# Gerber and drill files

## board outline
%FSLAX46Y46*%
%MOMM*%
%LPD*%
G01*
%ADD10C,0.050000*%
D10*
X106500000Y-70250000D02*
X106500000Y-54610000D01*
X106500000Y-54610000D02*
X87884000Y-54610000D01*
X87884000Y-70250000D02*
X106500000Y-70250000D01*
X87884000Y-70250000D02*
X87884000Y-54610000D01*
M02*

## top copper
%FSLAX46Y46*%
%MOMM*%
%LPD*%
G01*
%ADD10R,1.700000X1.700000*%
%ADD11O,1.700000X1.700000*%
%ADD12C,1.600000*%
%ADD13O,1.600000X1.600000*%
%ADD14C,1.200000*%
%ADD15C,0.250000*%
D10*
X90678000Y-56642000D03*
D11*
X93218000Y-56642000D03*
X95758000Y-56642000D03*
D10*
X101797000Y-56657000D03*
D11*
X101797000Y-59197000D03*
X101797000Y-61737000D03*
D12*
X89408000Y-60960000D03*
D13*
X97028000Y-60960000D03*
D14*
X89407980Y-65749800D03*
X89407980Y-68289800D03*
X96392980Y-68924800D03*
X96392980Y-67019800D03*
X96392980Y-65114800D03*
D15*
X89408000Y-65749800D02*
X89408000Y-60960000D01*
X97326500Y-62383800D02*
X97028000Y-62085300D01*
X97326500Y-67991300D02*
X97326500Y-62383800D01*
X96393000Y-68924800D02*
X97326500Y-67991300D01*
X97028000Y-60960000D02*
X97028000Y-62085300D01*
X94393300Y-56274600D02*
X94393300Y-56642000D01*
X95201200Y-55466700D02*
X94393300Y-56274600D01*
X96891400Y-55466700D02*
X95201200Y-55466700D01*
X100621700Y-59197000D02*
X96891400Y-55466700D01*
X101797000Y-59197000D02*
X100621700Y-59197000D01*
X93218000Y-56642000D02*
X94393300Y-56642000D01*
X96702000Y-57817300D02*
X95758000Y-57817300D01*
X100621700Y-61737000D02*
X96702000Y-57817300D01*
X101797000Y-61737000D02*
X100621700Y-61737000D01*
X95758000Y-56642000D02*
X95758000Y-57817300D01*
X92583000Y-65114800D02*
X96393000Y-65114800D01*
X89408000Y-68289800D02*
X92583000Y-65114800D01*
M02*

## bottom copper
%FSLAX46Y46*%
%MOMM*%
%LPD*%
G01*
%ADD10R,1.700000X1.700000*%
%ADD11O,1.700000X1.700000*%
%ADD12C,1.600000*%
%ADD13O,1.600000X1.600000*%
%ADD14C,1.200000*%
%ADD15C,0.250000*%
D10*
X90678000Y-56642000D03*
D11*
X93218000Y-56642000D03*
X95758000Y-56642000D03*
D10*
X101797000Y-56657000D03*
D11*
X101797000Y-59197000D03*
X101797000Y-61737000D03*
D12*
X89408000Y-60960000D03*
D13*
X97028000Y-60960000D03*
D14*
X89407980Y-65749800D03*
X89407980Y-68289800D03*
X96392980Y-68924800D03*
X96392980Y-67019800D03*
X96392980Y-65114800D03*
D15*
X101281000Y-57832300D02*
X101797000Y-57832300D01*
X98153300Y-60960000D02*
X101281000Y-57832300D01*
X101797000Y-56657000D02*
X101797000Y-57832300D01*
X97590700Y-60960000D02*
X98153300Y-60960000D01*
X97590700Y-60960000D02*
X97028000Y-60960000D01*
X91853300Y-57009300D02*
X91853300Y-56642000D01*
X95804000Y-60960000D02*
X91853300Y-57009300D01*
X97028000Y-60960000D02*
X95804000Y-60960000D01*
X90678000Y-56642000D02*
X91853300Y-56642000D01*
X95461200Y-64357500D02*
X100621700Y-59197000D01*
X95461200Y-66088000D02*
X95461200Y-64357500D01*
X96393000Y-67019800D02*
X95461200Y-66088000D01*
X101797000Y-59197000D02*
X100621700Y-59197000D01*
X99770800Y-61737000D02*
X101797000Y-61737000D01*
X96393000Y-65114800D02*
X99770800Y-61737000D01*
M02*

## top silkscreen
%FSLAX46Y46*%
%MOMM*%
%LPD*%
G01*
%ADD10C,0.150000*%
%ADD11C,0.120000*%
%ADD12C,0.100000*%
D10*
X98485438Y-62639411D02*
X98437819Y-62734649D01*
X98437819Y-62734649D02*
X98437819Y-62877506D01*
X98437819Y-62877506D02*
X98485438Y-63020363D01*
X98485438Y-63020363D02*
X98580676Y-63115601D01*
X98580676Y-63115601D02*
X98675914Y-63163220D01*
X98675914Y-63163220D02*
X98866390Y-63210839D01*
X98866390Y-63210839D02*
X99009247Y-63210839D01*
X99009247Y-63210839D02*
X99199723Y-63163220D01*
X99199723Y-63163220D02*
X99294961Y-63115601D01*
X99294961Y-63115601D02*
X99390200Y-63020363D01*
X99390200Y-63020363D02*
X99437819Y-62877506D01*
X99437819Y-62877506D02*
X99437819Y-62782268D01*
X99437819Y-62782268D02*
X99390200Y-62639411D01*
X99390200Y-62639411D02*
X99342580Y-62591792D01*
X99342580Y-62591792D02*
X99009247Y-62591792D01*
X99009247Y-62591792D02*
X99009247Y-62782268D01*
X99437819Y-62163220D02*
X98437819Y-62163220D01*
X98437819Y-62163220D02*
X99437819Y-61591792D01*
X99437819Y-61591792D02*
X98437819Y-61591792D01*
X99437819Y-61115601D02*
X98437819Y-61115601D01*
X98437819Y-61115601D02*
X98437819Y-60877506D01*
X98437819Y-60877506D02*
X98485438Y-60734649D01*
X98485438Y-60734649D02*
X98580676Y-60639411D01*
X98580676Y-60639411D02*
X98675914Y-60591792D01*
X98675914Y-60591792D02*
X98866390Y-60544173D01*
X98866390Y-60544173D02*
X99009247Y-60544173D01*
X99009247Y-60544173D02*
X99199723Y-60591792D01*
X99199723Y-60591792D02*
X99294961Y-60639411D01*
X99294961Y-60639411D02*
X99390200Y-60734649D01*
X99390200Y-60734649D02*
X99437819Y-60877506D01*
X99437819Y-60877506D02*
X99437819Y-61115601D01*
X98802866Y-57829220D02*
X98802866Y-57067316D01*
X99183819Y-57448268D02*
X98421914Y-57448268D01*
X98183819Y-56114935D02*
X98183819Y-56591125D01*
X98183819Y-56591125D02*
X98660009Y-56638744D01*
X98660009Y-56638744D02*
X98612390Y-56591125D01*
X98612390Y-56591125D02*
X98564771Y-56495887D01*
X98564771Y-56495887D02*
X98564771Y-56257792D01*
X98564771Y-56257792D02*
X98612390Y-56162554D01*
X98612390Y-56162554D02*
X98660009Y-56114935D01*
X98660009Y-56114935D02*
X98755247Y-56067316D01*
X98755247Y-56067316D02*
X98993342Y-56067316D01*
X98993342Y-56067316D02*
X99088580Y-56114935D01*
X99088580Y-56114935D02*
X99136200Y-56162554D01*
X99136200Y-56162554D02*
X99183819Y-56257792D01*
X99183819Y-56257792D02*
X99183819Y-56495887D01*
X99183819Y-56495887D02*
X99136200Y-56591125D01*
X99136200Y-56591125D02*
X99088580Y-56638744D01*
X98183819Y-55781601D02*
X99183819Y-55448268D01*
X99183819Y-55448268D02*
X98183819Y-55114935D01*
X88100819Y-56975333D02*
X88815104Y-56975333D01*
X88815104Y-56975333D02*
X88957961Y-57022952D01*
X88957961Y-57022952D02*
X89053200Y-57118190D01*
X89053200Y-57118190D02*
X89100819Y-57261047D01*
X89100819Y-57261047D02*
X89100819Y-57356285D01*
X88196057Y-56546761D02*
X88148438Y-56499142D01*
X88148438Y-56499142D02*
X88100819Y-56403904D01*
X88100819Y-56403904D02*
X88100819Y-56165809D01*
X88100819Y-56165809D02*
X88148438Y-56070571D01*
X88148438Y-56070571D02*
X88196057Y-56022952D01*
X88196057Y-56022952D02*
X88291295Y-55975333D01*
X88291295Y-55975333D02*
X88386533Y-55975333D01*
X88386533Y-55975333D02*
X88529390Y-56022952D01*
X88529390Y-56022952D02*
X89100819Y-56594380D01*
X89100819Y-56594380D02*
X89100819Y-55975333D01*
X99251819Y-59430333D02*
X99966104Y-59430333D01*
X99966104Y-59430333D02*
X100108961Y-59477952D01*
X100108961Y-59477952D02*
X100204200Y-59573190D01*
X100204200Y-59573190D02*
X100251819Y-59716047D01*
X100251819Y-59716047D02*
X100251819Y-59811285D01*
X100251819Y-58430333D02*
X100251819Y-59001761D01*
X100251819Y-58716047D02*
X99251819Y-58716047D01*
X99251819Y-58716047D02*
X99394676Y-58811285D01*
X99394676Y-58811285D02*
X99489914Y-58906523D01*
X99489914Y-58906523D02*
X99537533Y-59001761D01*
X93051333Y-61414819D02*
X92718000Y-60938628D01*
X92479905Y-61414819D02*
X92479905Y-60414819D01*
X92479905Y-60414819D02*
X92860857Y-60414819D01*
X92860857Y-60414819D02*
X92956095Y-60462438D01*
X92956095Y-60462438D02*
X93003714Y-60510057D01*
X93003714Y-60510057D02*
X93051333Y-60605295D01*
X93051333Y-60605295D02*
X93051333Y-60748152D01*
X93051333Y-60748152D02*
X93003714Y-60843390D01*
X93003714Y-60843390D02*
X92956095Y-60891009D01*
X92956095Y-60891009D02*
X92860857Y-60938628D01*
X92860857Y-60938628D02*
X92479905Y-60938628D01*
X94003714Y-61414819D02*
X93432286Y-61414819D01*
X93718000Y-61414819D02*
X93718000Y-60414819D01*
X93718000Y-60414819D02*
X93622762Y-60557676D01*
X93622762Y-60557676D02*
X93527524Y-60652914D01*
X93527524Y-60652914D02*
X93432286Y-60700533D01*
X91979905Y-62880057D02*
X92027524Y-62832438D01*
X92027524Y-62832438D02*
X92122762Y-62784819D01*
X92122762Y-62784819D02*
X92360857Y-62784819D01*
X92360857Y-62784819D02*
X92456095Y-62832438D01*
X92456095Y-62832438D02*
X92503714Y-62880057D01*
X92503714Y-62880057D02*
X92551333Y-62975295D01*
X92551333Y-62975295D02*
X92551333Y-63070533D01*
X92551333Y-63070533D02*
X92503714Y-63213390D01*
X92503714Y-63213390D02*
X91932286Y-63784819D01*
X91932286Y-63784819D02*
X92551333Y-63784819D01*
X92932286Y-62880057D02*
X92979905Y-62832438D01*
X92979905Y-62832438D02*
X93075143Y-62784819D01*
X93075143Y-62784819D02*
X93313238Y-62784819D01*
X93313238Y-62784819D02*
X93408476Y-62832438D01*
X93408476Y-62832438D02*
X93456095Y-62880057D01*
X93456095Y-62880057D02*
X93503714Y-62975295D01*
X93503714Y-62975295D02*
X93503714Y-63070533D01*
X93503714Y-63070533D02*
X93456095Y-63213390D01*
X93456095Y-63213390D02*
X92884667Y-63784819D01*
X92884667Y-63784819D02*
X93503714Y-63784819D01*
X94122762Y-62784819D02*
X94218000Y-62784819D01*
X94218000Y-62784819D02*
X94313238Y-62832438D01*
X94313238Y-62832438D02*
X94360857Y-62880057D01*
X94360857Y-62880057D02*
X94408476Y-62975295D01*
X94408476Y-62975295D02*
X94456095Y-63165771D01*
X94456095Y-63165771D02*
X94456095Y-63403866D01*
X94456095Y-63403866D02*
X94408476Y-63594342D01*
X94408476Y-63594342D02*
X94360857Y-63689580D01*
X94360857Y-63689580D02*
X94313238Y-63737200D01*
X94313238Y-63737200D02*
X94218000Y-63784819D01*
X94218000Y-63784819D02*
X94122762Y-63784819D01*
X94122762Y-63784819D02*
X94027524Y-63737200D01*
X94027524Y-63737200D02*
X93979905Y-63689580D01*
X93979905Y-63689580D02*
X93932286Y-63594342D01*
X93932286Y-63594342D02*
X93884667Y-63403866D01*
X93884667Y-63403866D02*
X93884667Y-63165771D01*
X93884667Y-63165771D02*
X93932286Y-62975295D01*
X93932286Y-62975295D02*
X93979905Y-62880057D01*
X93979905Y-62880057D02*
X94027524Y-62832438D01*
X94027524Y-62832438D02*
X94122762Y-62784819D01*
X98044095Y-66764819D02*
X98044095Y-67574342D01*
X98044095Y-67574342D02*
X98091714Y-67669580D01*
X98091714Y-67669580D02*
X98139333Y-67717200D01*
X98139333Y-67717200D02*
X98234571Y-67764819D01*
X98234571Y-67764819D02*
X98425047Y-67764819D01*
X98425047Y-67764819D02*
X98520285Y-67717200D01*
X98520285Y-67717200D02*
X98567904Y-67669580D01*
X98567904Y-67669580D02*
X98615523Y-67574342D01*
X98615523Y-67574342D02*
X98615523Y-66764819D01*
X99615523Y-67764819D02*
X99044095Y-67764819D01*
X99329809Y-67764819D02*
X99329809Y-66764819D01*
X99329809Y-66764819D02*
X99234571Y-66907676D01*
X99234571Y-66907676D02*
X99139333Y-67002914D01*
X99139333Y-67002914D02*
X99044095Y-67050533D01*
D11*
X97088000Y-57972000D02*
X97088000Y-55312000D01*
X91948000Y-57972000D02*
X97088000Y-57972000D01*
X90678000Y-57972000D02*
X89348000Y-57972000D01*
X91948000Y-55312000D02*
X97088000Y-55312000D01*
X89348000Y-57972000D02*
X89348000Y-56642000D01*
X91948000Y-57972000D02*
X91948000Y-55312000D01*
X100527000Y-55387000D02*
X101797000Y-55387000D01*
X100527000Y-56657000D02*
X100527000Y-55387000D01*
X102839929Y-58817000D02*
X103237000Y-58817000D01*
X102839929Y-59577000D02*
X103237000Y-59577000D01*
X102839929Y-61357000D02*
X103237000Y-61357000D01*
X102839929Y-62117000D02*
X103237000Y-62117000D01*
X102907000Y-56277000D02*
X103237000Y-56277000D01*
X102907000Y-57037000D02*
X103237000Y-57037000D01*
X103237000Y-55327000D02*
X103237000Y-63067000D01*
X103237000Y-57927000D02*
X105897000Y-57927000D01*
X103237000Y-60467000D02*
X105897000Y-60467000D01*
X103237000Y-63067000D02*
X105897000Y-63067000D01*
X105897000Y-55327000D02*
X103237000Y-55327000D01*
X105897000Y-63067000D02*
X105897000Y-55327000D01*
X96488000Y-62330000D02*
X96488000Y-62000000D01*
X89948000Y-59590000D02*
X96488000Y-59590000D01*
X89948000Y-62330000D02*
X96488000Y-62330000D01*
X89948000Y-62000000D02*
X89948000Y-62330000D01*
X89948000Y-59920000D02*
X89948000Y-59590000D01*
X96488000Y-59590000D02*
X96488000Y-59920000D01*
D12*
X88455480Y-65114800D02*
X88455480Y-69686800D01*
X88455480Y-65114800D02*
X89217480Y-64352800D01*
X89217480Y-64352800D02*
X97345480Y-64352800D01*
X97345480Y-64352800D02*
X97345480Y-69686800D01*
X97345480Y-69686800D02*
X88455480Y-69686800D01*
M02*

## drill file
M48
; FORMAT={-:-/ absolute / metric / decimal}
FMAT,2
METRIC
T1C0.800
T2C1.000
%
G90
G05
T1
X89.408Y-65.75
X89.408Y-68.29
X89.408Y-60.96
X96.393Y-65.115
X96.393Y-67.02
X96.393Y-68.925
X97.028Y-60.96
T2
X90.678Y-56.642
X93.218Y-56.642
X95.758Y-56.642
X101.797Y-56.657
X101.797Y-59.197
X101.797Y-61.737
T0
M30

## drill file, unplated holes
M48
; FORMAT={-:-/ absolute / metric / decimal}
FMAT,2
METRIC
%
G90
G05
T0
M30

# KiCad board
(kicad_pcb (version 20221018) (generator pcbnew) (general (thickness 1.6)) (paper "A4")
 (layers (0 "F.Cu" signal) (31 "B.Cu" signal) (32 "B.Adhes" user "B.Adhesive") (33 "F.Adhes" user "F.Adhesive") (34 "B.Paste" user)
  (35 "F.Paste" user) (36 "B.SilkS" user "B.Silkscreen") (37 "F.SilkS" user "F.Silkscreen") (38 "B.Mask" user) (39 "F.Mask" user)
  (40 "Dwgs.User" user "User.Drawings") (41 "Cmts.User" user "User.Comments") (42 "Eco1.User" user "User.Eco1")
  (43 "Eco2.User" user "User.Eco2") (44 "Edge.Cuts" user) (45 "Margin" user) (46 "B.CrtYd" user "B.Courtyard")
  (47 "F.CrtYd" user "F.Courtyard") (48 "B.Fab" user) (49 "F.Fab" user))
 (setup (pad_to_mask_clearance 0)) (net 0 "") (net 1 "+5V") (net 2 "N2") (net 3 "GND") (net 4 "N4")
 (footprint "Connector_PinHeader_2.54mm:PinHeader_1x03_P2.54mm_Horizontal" (layer "F.Cu") (at 101.797 56.657)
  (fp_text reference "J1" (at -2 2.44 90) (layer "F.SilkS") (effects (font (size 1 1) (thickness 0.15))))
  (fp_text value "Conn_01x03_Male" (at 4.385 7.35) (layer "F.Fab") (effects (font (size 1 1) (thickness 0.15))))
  (fp_line (start -1.27 -1.27) (end 0 -1.27) (stroke (width 0.12) (type solid)) (layer "F.SilkS"))
  (fp_line (start -1.27 0) (end -1.27 -1.27) (stroke (width 0.12) (type solid)) (layer "F.SilkS"))
  (fp_line (start 1.042929 2.16) (end 1.44 2.16) (stroke (width 0.12) (type solid)) (layer "F.SilkS"))
  (fp_line (start 1.042929 2.92) (end 1.44 2.92) (stroke (width 0.12) (type solid)) (layer "F.SilkS"))
  (fp_line (start 1.042929 4.7) (end 1.44 4.7) (stroke (width 0.12) (type solid)) (layer "F.SilkS"))
  (fp_line (start 1.042929 5.46) (end 1.44 5.46) (stroke (width 0.12) (type solid)) (layer "F.SilkS"))
  (fp_line (start 1.11 -0.38) (end 1.44 -0.38) (stroke (width 0.12) (type solid)) (layer "F.SilkS"))
  (fp_line (start 1.11 0.38) (end 1.44 0.38) (stroke (width 0.12) (type solid)) (layer "F.SilkS"))
  (fp_line (start 1.44 -1.33) (end 1.44 6.41) (stroke (width 0.12) (type solid)) (layer "F.SilkS"))
  (fp_line (start 1.44 1.27) (end 4.1 1.27) (stroke (width 0.12) (type solid)) (layer "F.SilkS"))
  (fp_line (start 1.44 3.81) (end 4.1 3.81) (stroke (width 0.12) (type solid)) (layer "F.SilkS"))
  (fp_line (start 1.44 6.41) (end 4.1 6.41) (stroke (width 0.12) (type solid)) (layer "F.SilkS"))
  (fp_line (start 4.1 -1.33) (end 1.44 -1.33) (stroke (width 0.12) (type solid)) (layer "F.SilkS"))
  (fp_line (start 4.1 6.41) (end 4.1 -1.33) (stroke (width 0.12) (type solid)) (layer "F.SilkS"))
  (pad "1" thru_hole rect (at 0 0) (size 1.7 1.7) (drill 1) (layers "*.Cu" "*.Mask") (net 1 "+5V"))
  (pad "2" thru_hole oval (at 0 2.54) (size 1.7 1.7) (drill 1) (layers "*.Cu" "*.Mask") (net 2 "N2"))
  (pad "3" thru_hole oval (at 0 5.08) (size 1.7 1.7) (drill 1) (layers "*.Cu" "*.Mask") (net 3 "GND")))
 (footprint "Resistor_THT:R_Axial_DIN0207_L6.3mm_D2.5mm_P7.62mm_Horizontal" (layer "F.Cu") (at 89.408 60.96)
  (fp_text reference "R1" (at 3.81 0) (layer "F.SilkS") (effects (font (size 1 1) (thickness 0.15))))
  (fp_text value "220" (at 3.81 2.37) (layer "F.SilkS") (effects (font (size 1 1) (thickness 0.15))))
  (fp_line (start 0.54 -1.37) (end 7.08 -1.37) (stroke (width 0.12) (type solid)) (layer "F.SilkS"))
  (fp_line (start 0.54 -1.04) (end 0.54 -1.37) (stroke (width 0.12) (type solid)) (layer "F.SilkS"))
  (fp_line (start 0.54 1.04) (end 0.54 1.37) (stroke (width 0.12) (type solid)) (layer "F.SilkS"))
  (fp_line (start 0.54 1.37) (end 7.08 1.37) (stroke (width 0.12) (type solid)) (layer "F.SilkS"))
  (fp_line (start 7.08 -1.37) (end 7.08 -1.04) (stroke (width 0.12) (type solid)) (layer "F.SilkS"))
  (fp_line (start 7.08 1.37) (end 7.08 1.04) (stroke (width 0.12) (type solid)) (layer "F.SilkS"))
  (pad "1" thru_hole circle (at 0 0) (size 1.6 1.6) (drill 0.8) (layers "*.Cu" "*.Mask") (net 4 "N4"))
  (pad "2" thru_hole oval (at 7.62 0) (size 1.6 1.6) (drill 0.8) (layers "*.Cu" "*.Mask") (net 1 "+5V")))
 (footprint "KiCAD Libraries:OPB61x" (layer "F.Cu") (at 89.4078 65.75)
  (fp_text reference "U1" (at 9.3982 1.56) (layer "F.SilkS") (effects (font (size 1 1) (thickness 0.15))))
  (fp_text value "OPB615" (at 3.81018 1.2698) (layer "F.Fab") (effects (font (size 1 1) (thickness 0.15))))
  (fp_line (start -0.95232 -0.6352) (end -0.95232 3.9368) (stroke (width 0.1) (type solid)) (layer "F.SilkS"))
  (fp_line (start -0.95232 -0.6352) (end -0.19032 -1.3972) (stroke (width 0.1) (type solid)) (layer "F.SilkS"))
  (fp_line (start -0.19032 -1.3972) (end 7.93768 -1.3972) (stroke (width 0.1) (type solid)) (layer "F.SilkS"))
  (fp_line (start 7.93768 -1.3972) (end 7.93768 3.9368) (stroke (width 0.1) (type solid)) (layer "F.SilkS"))
  (fp_line (start 7.93768 3.9368) (end -0.95232 3.9368) (stroke (width 0.1) (type solid)) (layer "F.SilkS"))
  (pad "1" thru_hole circle (at 0.00018 -0.0002) (size 1.2 1.2) (drill 0.8) (layers "*.Cu" "*.Mask") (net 4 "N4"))
  (pad "2" thru_hole circle (at 0.00018 2.5398) (size 1.2 1.2) (drill 0.8) (layers "*.Cu" "*.Mask") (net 3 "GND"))
  (pad "3" thru_hole circle (at 6.98518 3.1748) (size 1.2 1.2) (drill 0.8) (layers "*.Cu" "*.Mask") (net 1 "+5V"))
  (pad "4" thru_hole circle (at 6.98518 1.2698) (size 1.2 1.2) (drill 0.8) (layers "*.Cu" "*.Mask") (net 2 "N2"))
  (pad "5" thru_hole circle (at 6.98518 -0.6352) (size 1.2 1.2) (drill 0.8) (layers "*.Cu" "*.Mask") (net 3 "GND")))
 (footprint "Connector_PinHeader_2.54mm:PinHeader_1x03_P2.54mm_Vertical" (layer "F.Cu") (at 90.678 56.642 90)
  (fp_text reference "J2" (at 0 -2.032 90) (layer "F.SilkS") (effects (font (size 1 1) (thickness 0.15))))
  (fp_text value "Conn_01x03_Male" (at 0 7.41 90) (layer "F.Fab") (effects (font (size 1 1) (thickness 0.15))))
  (fp_line (start -1.33 -1.33) (end 0 -1.33) (stroke (width 0.12) (type solid)) (layer "F.SilkS"))
  (fp_line (start -1.33 0) (end -1.33 -1.33) (stroke (width 0.12) (type solid)) (layer "F.SilkS"))
  (fp_line (start -1.33 1.27) (end -1.33 6.41) (stroke (width 0.12) (type solid)) (layer "F.SilkS"))
  (fp_line (start -1.33 1.27) (end 1.33 1.27) (stroke (width 0.12) (type solid)) (layer "F.SilkS"))
  (fp_line (start -1.33 6.41) (end 1.33 6.41) (stroke (width 0.12) (type solid)) (layer "F.SilkS"))
  (fp_line (start 1.33 1.27) (end 1.33 6.41) (stroke (width 0.12) (type solid)) (layer "F.SilkS"))
  (pad "1" thru_hole rect (at 0 0 90) (size 1.7 1.7) (drill 1) (layers "*.Cu" "*.Mask") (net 1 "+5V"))
  (pad "2" thru_hole oval (at 0 2.54 90) (size 1.7 1.7) (drill 1) (layers "*.Cu" "*.Mask") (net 2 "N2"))
  (pad "3" thru_hole oval (at 0 5.08 90) (size 1.7 1.7) (drill 1) (layers "*.Cu" "*.Mask") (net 3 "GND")))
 (gr_line (start 106.5 70.25) (end 106.5 54.61) (stroke (width 0.05) (type solid)) (layer "Edge.Cuts"))
 (gr_line (start 106.5 54.61) (end 87.884 54.61) (stroke (width 0.05) (type solid)) (layer "Edge.Cuts"))
 (gr_line (start 87.884 70.25) (end 106.5 70.25) (stroke (width 0.05) (type solid)) (layer "Edge.Cuts"))
 (gr_line (start 87.884 70.25) (end 87.884 54.61) (stroke (width 0.05) (type solid)) (layer "Edge.Cuts"))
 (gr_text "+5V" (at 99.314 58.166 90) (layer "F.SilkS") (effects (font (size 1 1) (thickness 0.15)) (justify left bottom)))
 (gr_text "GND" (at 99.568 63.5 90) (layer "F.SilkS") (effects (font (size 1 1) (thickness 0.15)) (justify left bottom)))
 (segment (start 95.758 56.642) (end 95.758 57.8173) (width 0.25) (layer "F.Cu") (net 3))
 (segment (start 101.797 61.737) (end 100.6217 61.737) (width 0.25) (layer "F.Cu") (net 3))
 (segment (start 96.702 57.8173) (end 95.758 57.8173) (width 0.25) (layer "F.Cu") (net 3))
 (segment (start 89.408 68.2898) (end 92.583 65.1148) (width 0.25) (layer "F.Cu") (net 3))
 (segment (start 92.583 65.1148) (end 96.393 65.1148) (width 0.25) (layer "F.Cu") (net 3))
 (segment (start 100.6217 61.737) (end 96.702 57.8173) (width 0.25) (layer "F.Cu") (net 3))
 (segment (start 99.7708 61.737) (end 101.797 61.737) (width 0.25) (layer "B.Cu") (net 3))
 (segment (start 96.393 65.1148) (end 99.7708 61.737) (width 0.25) (layer "B.Cu") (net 3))
 (segment (start 94.3933 56.2746) (end 94.3933 56.642) (width 0.25) (layer "F.Cu") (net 2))
 (segment (start 96.8914 55.4667) (end 95.2012 55.4667) (width 0.25) (layer "F.Cu") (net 2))
 (segment (start 93.218 56.642) (end 94.3933 56.642) (width 0.25) (layer "F.Cu") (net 2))
 (segment (start 100.6217 59.197) (end 96.8914 55.4667) (width 0.25) (layer "F.Cu") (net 2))
 (segment (start 95.2012 55.4667) (end 94.3933 56.2746) (width 0.25) (layer "F.Cu") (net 2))
 (segment (start 101.797 59.197) (end 100.6217 59.197) (width 0.25) (layer "F.Cu") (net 2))
 (segment (start 101.797 59.197) (end 100.6217 59.197) (width 0.25) (layer "B.Cu") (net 2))
 (segment (start 95.4612 64.3575) (end 100.6217 59.197) (width 0.25) (layer "B.Cu") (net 2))
 (segment (start 95.4612 66.088) (end 95.4612 64.3575) (width 0.25) (layer "B.Cu") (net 2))
 (segment (start 96.393 67.0198) (end 95.4612 66.088) (width 0.25) (layer "B.Cu") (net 2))
 (segment (start 96.393 68.9248) (end 97.3265 67.9913) (width 0.25) (layer "F.Cu") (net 1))
 (segment (start 97.028 60.96) (end 97.028 62.0853) (width 0.25) (layer "F.Cu") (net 1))
 (segment (start 97.3265 67.9913) (end 97.3265 62.3838) (width 0.25) (layer "F.Cu") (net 1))
 (segment (start 97.3265 62.3838) (end 97.028 62.0853) (width 0.25) (layer "F.Cu") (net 1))
 (segment (start 91.8533 57.0093) (end 91.8533 56.642) (width 0.25) (layer "B.Cu") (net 1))
 (segment (start 97.5907 60.96) (end 97.028 60.96) (width 0.25) (layer "B.Cu") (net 1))
 (segment (start 90.678 56.642) (end 91.8533 56.642) (width 0.25) (layer "B.Cu") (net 1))
 (segment (start 97.5907 60.96) (end 98.1533 60.96) (width 0.25) (layer "B.Cu") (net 1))
 (segment (start 97.028 60.96) (end 95.804 60.96) (width 0.25) (layer "B.Cu") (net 1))
 (segment (start 95.804 60.96) (end 91.8533 57.0093) (width 0.25) (layer "B.Cu") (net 1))
 (segment (start 101.281 57.8323) (end 101.797 57.8323) (width 0.25) (layer "B.Cu") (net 1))
 (segment (start 98.1533 60.96) (end 101.281 57.8323) (width 0.25) (layer "B.Cu") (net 1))
 (segment (start 101.797 56.657) (end 101.797 57.8323) (width 0.25) (layer "B.Cu") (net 1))
 (segment (start 89.408 65.7498) (end 89.408 60.96) (width 0.25) (layer "F.Cu") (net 4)))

